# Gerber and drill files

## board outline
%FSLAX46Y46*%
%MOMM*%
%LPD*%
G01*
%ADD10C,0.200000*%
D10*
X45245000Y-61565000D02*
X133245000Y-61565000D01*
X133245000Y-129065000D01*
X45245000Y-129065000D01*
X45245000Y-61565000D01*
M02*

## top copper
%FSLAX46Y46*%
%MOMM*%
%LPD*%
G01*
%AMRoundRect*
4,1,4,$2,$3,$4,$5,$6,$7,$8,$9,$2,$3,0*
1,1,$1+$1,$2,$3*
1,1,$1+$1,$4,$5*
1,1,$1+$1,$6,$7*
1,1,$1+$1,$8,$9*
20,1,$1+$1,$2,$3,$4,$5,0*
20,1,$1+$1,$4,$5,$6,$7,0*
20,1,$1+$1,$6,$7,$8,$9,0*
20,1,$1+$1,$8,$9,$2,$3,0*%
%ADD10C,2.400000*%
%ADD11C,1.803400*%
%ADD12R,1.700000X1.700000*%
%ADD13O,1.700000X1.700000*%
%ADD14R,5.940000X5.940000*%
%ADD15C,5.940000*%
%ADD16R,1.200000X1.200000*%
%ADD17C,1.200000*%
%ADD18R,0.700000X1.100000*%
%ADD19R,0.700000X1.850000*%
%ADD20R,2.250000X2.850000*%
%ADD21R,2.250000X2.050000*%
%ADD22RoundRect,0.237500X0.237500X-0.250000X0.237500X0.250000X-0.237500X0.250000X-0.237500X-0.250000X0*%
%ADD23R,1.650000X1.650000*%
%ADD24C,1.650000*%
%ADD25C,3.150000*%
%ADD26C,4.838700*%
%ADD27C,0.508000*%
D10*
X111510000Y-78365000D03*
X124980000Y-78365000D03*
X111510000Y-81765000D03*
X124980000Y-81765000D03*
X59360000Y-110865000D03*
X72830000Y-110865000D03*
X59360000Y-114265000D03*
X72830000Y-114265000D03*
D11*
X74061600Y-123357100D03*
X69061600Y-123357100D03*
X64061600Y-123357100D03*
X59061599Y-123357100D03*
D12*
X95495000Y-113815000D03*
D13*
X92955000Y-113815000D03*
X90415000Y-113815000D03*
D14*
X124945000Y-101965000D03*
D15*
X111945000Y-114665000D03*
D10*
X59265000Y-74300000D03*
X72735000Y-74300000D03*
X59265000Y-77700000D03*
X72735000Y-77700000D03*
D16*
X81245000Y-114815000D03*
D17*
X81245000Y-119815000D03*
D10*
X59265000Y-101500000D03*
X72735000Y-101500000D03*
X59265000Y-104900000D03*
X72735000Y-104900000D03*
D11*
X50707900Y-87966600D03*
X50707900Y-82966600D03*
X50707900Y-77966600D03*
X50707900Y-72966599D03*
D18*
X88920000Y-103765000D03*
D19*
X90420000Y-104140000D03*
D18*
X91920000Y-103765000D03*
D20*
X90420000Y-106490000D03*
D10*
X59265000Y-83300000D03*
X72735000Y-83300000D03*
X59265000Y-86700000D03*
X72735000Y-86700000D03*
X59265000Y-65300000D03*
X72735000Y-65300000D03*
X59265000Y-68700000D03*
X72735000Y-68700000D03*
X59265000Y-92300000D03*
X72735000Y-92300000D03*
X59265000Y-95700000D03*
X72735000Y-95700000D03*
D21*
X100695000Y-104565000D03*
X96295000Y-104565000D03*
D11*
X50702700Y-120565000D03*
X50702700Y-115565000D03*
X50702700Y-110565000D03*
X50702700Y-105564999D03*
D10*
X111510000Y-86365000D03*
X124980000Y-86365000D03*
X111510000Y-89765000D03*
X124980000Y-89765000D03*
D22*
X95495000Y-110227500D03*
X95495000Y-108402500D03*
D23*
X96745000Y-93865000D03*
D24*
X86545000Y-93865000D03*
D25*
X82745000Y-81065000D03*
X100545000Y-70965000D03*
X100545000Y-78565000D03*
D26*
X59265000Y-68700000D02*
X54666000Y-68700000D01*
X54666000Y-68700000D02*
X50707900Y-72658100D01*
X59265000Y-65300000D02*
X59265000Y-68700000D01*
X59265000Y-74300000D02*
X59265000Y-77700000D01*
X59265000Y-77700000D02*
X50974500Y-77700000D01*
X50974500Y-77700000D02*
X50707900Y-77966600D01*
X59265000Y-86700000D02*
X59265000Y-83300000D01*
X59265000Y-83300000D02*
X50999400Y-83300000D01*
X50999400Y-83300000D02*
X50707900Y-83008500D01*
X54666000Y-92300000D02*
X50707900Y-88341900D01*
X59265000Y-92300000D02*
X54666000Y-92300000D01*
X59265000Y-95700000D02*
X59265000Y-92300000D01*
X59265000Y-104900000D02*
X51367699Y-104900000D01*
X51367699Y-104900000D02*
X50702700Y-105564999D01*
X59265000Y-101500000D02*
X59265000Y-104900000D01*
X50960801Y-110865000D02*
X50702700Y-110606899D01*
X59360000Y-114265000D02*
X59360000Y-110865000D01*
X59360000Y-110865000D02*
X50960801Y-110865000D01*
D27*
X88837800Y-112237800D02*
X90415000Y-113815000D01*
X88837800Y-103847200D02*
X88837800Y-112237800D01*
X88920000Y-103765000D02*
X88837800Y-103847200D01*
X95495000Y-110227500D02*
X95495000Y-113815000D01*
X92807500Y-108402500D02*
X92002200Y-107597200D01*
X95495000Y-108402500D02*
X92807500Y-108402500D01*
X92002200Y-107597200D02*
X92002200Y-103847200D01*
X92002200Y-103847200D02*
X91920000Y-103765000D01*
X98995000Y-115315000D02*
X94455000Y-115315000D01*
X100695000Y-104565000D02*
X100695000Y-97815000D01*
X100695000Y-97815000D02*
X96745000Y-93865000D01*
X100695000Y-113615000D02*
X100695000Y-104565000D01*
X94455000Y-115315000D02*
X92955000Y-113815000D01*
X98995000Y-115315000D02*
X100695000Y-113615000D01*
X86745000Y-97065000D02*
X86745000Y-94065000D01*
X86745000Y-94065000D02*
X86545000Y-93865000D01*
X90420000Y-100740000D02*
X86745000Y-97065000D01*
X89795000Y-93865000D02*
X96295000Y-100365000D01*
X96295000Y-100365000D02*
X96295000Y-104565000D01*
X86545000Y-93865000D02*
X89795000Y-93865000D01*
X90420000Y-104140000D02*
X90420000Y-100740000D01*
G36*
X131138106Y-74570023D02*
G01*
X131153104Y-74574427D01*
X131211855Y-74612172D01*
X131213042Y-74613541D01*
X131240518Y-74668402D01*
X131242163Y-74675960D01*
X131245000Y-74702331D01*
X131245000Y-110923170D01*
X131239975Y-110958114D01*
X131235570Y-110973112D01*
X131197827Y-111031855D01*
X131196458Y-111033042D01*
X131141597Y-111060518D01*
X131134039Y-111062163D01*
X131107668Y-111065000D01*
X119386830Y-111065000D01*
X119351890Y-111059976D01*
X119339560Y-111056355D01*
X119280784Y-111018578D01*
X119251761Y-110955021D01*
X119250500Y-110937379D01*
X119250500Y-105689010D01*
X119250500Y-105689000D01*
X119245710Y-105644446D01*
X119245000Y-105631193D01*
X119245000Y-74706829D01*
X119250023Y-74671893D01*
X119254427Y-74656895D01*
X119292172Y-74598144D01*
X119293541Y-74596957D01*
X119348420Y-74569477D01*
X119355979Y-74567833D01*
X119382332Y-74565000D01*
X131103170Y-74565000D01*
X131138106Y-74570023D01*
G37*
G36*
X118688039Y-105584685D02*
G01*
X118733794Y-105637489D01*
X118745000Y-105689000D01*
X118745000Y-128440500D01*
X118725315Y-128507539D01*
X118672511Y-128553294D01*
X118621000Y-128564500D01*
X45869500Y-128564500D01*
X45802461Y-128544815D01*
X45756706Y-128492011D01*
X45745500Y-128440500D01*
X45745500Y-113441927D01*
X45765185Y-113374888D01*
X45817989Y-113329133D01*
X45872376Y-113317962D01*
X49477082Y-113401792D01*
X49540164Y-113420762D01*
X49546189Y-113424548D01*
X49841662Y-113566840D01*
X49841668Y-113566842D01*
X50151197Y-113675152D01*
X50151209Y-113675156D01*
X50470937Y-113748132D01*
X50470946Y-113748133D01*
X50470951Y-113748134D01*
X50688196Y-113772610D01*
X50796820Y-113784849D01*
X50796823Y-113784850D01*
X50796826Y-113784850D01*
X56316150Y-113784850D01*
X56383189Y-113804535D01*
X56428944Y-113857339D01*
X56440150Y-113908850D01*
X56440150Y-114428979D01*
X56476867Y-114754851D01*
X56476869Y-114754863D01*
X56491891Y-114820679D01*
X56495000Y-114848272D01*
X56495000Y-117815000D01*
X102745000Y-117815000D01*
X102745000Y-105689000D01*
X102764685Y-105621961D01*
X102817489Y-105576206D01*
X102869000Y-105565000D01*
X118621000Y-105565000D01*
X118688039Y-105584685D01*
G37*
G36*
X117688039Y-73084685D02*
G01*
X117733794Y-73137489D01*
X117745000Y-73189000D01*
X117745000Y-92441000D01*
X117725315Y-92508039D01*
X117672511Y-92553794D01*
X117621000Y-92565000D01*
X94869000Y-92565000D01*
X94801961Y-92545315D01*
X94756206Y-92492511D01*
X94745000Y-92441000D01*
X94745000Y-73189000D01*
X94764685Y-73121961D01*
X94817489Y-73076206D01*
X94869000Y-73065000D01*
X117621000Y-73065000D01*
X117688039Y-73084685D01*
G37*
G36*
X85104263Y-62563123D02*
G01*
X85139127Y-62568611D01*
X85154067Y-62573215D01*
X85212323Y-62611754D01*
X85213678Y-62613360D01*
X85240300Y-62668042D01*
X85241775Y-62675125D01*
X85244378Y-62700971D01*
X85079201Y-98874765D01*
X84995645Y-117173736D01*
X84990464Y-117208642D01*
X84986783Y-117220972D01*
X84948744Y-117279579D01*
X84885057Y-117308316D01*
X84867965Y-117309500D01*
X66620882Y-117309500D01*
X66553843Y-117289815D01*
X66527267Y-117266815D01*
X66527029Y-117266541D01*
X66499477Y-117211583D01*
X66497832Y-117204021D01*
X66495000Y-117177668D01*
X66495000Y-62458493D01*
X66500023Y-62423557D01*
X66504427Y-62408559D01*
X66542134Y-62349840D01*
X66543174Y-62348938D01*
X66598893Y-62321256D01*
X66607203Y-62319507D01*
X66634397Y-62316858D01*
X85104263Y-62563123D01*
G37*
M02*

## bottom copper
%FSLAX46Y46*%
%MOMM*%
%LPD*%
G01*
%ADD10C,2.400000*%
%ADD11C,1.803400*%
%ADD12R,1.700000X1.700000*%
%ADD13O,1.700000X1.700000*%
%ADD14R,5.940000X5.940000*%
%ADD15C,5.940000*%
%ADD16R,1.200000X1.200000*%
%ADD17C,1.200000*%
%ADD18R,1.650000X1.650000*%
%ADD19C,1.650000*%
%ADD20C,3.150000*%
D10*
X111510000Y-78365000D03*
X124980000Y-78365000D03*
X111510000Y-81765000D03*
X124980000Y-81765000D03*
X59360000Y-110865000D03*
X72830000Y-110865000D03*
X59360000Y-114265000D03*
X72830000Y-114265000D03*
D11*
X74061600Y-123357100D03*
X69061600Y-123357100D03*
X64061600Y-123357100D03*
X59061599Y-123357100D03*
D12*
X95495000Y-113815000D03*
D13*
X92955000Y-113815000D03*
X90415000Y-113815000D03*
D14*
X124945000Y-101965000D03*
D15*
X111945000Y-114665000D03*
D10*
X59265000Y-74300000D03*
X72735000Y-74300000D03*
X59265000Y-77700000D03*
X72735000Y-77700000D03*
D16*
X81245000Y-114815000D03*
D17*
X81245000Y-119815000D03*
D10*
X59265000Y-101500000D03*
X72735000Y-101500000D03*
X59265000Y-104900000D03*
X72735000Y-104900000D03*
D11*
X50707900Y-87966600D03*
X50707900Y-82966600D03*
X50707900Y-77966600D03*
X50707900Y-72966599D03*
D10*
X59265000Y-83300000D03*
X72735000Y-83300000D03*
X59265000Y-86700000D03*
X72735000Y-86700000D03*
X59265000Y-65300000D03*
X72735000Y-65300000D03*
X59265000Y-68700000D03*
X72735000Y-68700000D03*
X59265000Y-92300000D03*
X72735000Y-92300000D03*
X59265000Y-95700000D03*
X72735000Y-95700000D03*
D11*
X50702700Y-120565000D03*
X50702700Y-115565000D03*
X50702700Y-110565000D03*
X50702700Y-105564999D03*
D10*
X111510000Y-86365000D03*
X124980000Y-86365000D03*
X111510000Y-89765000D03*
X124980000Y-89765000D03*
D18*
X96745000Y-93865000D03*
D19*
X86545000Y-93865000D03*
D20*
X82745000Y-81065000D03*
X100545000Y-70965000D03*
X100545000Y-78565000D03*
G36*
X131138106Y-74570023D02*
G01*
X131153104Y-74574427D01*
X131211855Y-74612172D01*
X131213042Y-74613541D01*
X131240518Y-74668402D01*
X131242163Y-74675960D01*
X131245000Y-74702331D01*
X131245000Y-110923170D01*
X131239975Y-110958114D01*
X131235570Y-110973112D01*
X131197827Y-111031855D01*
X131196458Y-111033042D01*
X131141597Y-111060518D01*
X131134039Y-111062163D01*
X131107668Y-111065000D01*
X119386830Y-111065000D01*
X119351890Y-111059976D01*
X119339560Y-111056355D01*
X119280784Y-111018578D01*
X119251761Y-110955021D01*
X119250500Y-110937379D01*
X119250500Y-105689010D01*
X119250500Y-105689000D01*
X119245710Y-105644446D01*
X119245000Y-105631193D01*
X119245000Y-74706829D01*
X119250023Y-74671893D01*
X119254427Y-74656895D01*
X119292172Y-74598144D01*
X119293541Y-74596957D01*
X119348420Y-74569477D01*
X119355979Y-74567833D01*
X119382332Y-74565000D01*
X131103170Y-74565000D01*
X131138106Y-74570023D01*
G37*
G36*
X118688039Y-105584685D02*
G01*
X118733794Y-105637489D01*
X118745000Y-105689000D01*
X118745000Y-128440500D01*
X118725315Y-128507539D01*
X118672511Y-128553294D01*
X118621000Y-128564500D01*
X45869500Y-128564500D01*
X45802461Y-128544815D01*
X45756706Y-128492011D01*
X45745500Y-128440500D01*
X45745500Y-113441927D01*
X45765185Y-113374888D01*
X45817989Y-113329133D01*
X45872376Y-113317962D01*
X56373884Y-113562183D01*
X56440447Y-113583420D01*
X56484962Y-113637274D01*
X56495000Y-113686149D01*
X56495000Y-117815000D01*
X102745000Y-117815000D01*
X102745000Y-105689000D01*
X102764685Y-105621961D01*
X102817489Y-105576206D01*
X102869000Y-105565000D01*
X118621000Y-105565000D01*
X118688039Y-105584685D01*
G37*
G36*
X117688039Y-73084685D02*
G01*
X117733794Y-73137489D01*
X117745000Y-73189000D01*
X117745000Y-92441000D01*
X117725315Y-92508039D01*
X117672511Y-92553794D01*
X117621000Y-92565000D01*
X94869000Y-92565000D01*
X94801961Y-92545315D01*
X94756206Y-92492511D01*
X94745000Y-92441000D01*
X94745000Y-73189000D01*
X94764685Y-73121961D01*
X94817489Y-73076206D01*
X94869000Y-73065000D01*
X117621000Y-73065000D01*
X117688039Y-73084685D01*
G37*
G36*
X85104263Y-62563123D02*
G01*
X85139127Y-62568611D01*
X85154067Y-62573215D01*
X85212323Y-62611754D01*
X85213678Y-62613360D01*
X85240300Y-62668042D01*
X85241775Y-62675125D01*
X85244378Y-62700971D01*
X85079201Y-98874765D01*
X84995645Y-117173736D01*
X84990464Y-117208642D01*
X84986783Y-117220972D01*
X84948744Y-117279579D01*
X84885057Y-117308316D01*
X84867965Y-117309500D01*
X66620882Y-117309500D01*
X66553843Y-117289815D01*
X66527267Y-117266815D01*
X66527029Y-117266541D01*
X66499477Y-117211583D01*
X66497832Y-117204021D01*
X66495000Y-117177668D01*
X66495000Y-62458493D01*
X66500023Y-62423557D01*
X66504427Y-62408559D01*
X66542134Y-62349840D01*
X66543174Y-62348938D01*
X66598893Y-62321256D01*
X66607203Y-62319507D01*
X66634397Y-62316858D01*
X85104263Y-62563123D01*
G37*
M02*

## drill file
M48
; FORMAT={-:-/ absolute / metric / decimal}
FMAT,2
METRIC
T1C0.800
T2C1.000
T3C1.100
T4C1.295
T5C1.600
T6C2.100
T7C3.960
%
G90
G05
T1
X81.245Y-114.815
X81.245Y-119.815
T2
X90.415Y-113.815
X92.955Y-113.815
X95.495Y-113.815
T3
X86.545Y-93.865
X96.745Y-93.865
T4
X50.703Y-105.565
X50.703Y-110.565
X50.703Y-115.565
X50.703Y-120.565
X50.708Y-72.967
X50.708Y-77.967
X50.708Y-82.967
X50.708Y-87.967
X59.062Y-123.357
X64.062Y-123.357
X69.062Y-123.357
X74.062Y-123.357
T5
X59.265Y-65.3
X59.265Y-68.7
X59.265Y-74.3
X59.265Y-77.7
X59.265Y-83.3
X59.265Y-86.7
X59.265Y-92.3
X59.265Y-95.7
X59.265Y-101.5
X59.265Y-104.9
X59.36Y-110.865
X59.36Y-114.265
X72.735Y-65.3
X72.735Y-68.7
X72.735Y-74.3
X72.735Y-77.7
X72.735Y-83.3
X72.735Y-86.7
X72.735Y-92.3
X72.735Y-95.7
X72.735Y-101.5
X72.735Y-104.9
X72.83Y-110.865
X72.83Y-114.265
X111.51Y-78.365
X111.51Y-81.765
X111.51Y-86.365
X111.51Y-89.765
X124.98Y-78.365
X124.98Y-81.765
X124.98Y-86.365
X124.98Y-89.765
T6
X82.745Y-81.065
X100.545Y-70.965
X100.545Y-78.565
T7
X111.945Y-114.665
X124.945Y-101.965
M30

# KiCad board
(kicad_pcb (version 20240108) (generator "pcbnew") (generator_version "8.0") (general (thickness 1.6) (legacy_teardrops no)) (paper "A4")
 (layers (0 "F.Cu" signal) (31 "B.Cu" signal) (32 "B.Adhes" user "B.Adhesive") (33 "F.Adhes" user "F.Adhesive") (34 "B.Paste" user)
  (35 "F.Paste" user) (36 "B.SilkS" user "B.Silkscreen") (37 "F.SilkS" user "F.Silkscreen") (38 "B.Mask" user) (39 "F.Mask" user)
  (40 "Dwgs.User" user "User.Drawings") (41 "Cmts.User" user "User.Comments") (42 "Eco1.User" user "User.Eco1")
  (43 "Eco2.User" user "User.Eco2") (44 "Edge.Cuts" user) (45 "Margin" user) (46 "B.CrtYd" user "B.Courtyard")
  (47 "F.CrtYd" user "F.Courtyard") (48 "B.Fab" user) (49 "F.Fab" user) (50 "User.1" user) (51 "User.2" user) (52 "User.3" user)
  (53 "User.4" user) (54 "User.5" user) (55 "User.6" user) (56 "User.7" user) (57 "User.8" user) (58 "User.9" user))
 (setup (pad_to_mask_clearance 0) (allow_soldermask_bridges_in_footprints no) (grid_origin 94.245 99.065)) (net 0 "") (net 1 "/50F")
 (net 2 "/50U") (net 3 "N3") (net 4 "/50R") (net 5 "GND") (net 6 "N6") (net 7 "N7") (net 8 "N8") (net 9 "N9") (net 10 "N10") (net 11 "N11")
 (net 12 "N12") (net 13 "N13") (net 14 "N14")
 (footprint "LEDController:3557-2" (layer "F.Cu") (at 118.245 80.065)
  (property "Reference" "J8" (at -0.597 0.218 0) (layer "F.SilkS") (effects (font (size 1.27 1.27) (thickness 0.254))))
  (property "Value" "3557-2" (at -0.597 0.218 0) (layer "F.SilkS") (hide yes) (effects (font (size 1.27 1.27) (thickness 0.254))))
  (pad "1" thru_hole circle (at -6.735 -1.7) (size 2.4 2.4) (drill 1.6) (layers "*.Cu" "*.Mask") (remove_unused_layers no) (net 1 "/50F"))
  (pad "2" thru_hole circle (at 6.735 -1.7) (size 2.4 2.4) (drill 1.6) (layers "*.Cu" "*.Mask") (remove_unused_layers no) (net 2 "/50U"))
  (pad "3" thru_hole circle (at -6.735 1.7) (size 2.4 2.4) (drill 1.6) (layers "*.Cu" "*.Mask") (remove_unused_layers no) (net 1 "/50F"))
  (pad "4" thru_hole circle (at 6.735 1.7) (size 2.4 2.4) (drill 1.6) (layers "*.Cu" "*.Mask") (remove_unused_layers no) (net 2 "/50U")))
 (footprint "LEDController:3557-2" (layer "F.Cu") (at 66.095 112.565)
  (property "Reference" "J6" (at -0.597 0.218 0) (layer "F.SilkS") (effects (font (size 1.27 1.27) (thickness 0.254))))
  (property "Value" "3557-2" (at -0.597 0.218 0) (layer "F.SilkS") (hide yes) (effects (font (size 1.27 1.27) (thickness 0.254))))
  (pad "1" thru_hole circle (at -6.735 -1.7) (size 2.4 2.4) (drill 1.6) (layers "*.Cu" "*.Mask") (remove_unused_layers no) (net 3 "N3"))
  (pad "2" thru_hole circle (at 6.735 -1.7) (size 2.4 2.4) (drill 1.6) (layers "*.Cu" "*.Mask") (remove_unused_layers no) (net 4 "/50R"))
  (pad "3" thru_hole circle (at -6.735 1.7) (size 2.4 2.4) (drill 1.6) (layers "*.Cu" "*.Mask") (remove_unused_layers no) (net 3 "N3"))
  (pad "4" thru_hole circle (at 6.735 1.7) (size 2.4 2.4) (drill 1.6) (layers "*.Cu" "*.Mask") (remove_unused_layers no) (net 4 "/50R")))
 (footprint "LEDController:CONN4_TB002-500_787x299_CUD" (layer "F.Cu") (at 74.0616 123.3571)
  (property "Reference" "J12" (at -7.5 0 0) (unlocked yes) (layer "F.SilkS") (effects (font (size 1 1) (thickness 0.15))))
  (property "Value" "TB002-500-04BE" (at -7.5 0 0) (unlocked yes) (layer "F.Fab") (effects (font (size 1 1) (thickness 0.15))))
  (pad "1" thru_hole circle (at 0 0) (size 1.8034 1.8034) (drill 1.2954) (layers "*.Cu" "*.Mask") (remove_unused_layers no) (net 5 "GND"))
  (pad "2" thru_hole circle (at -5 0) (size 1.8034 1.8034) (drill 1.2954) (layers "*.Cu" "*.Mask") (remove_unused_layers no) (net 5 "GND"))
  (pad "3" thru_hole circle (at -10 0) (size 1.8034 1.8034) (drill 1.2954) (layers "*.Cu" "*.Mask") (remove_unused_layers no) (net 5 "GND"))
  (pad "4" thru_hole circle (at -15.000001 0) (size 1.8034 1.8034) (drill 1.2954) (layers "*.Cu" "*.Mask") (remove_unused_layers no)
   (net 5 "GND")))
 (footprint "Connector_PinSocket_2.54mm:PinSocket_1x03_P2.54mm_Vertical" (layer "F.Cu") (at 95.495 113.815 -90)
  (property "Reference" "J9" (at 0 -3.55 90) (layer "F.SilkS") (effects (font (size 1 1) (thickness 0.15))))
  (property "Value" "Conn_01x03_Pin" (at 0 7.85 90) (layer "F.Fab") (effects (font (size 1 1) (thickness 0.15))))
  (pad "1" thru_hole rect (at 0 0 270) (size 1.7 1.7) (drill 1) (layers "*.Cu" "*.Mask") (remove_unused_layers no) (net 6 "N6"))
  (pad "2" thru_hole oval (at 0 2.54 270) (size 1.7 1.7) (drill 1) (layers "*.Cu" "*.Mask") (remove_unused_layers no) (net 1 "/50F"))
  (pad "3" thru_hole oval (at 0 5.08 270) (size 1.7 1.7) (drill 1) (layers "*.Cu" "*.Mask") (remove_unused_layers no) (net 5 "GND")))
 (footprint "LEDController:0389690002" (layer "F.Cu") (at 124.945 101.965 -90)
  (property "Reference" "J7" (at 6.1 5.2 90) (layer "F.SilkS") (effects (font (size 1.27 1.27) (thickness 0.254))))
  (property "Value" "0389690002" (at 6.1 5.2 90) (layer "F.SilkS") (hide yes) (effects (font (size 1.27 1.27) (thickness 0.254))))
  (pad "1" thru_hole rect (at 0 0 270) (size 5.94 5.94) (drill 3.96) (layers "*.Cu" "*.Mask") (remove_unused_layers no) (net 2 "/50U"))
  (pad "2" thru_hole circle (at 12.7 13 270) (size 5.94 5.94) (drill 3.96) (layers "*.Cu" "*.Mask") (remove_unused_layers no) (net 5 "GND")))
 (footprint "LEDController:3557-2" (layer "F.Cu") (at 66 76)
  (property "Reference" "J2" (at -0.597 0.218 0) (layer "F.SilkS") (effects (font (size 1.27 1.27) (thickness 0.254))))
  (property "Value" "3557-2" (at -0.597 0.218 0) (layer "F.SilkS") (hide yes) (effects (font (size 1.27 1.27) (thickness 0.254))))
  (pad "1" thru_hole circle (at -6.735 -1.7) (size 2.4 2.4) (drill 1.6) (layers "*.Cu" "*.Mask") (remove_unused_layers no) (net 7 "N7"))
  (pad "2" thru_hole circle (at 6.735 -1.7) (size 2.4 2.4) (drill 1.6) (layers "*.Cu" "*.Mask") (remove_unused_layers no) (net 4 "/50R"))
  (pad "3" thru_hole circle (at -6.735 1.7) (size 2.4 2.4) (drill 1.6) (layers "*.Cu" "*.Mask") (remove_unused_layers no) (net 7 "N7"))
  (pad "4" thru_hole circle (at 6.735 1.7) (size 2.4 2.4) (drill 1.6) (layers "*.Cu" "*.Mask") (remove_unused_layers no) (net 4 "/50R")))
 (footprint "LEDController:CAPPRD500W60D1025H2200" (layer "F.Cu") (at 81.245 114.815 -90)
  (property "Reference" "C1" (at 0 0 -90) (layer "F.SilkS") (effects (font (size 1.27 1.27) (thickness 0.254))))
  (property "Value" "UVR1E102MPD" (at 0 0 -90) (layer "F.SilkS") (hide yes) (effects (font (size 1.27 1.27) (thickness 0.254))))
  (pad "1" thru_hole rect (at 0 0 270) (size 1.2 1.2) (drill 0.8) (layers "*.Cu" "*.Mask") (remove_unused_layers no) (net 4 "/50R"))
  (pad "2" thru_hole circle (at 5 0 270) (size 1.2 1.2) (drill 0.8) (layers "*.Cu" "*.Mask") (remove_unused_layers no) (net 5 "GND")))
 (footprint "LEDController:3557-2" (layer "F.Cu") (at 66 103.2)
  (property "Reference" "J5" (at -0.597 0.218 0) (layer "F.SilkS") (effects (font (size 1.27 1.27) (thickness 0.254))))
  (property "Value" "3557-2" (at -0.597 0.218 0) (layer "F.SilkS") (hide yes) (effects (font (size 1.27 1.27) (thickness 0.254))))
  (pad "1" thru_hole circle (at -6.735 -1.7) (size 2.4 2.4) (drill 1.6) (layers "*.Cu" "*.Mask") (remove_unused_layers no) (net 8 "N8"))
  (pad "2" thru_hole circle (at 6.735 -1.7) (size 2.4 2.4) (drill 1.6) (layers "*.Cu" "*.Mask") (remove_unused_layers no) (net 4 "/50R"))
  (pad "3" thru_hole circle (at -6.735 1.7) (size 2.4 2.4) (drill 1.6) (layers "*.Cu" "*.Mask") (remove_unused_layers no) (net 8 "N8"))
  (pad "4" thru_hole circle (at 6.735 1.7) (size 2.4 2.4) (drill 1.6) (layers "*.Cu" "*.Mask") (remove_unused_layers no) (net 4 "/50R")))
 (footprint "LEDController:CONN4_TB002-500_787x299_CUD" (layer "F.Cu") (at 50.7079 87.9666 -90)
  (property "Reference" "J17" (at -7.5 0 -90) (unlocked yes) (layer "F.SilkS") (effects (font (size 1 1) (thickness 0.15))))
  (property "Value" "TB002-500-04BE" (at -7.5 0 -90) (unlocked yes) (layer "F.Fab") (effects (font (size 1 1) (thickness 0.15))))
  (pad "1" thru_hole circle (at 0 0 270) (size 1.8034 1.8034) (drill 1.2954) (layers "*.Cu" "*.Mask") (remove_unused_layers no) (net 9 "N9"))
  (pad "2" thru_hole circle (at -5 0 270) (size 1.8034 1.8034) (drill 1.2954) (layers "*.Cu" "*.Mask") (remove_unused_layers no)
   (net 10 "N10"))
  (pad "3" thru_hole circle (at -10 0 270) (size 1.8034 1.8034) (drill 1.2954) (layers "*.Cu" "*.Mask") (remove_unused_layers no)
   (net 7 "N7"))
  (pad "4" thru_hole circle (at -15.000001 0 270) (size 1.8034 1.8034) (drill 1.2954) (layers "*.Cu" "*.Mask") (remove_unused_layers no)
   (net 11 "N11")))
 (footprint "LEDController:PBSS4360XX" (layer "F.Cu") (at 90.42 105.565 180)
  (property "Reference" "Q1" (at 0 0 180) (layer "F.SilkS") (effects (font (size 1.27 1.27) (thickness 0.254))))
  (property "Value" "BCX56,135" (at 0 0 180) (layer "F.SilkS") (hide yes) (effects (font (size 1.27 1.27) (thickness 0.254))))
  (pad "1" smd rect (at 1.5 1.8 180) (size 0.7 1.1) (layers "F.Cu" "F.Paste" "F.Mask") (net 5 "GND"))
  (pad "2" smd rect (at 0 1.425 180) (size 0.7 1.85) (layers "F.Cu" "F.Paste" "F.Mask") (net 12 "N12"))
  (pad "3" smd rect (at -1.5 1.8 180) (size 0.7 1.1) (layers "F.Cu" "F.Paste" "F.Mask") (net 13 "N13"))
  (pad "4" smd rect (at 0 -0.925 180) (size 2.25 2.85) (layers "F.Cu" "F.Paste" "F.Mask") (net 12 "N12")))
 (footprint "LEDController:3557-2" (layer "F.Cu") (at 66 85)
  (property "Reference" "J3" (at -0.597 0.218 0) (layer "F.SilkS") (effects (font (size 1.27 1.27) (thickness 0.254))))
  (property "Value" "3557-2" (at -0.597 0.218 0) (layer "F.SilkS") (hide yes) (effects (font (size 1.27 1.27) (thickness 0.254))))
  (pad "1" thru_hole circle (at -6.735 -1.7) (size 2.4 2.4) (drill 1.6) (layers "*.Cu" "*.Mask") (remove_unused_layers no) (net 10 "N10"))
  (pad "2" thru_hole circle (at 6.735 -1.7) (size 2.4 2.4) (drill 1.6) (layers "*.Cu" "*.Mask") (remove_unused_layers no) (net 4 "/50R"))
  (pad "3" thru_hole circle (at -6.735 1.7) (size 2.4 2.4) (drill 1.6) (layers "*.Cu" "*.Mask") (remove_unused_layers no) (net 10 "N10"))
  (pad "4" thru_hole circle (at 6.735 1.7) (size 2.4 2.4) (drill 1.6) (layers "*.Cu" "*.Mask") (remove_unused_layers no) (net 4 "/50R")))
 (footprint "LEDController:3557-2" (layer "F.Cu") (at 66 67)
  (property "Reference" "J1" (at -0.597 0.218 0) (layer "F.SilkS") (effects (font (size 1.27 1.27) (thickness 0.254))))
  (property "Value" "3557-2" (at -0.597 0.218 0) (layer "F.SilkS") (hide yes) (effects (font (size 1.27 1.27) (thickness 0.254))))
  (pad "1" thru_hole circle (at -6.735 -1.7) (size 2.4 2.4) (drill 1.6) (layers "*.Cu" "*.Mask") (remove_unused_layers no) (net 11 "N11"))
  (pad "2" thru_hole circle (at 6.735 -1.7) (size 2.4 2.4) (drill 1.6) (layers "*.Cu" "*.Mask") (remove_unused_layers no) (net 4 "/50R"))
  (pad "3" thru_hole circle (at -6.735 1.7) (size 2.4 2.4) (drill 1.6) (layers "*.Cu" "*.Mask") (remove_unused_layers no) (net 11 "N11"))
  (pad "4" thru_hole circle (at 6.735 1.7) (size 2.4 2.4) (drill 1.6) (layers "*.Cu" "*.Mask") (remove_unused_layers no) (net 4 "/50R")))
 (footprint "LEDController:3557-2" (layer "F.Cu") (at 66 94)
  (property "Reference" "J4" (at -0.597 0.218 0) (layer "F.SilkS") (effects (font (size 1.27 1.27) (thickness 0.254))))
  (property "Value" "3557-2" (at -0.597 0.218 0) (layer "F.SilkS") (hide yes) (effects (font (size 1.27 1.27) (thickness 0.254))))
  (pad "1" thru_hole circle (at -6.735 -1.7) (size 2.4 2.4) (drill 1.6) (layers "*.Cu" "*.Mask") (remove_unused_layers no) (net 9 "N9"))
  (pad "2" thru_hole circle (at 6.735 -1.7) (size 2.4 2.4) (drill 1.6) (layers "*.Cu" "*.Mask") (remove_unused_layers no) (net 4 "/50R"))
  (pad "3" thru_hole circle (at -6.735 1.7) (size 2.4 2.4) (drill 1.6) (layers "*.Cu" "*.Mask") (remove_unused_layers no) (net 9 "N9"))
  (pad "4" thru_hole circle (at 6.735 1.7) (size 2.4 2.4) (drill 1.6) (layers "*.Cu" "*.Mask") (remove_unused_layers no) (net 4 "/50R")))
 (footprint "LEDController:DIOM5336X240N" (layer "F.Cu") (at 98.495 104.565 180)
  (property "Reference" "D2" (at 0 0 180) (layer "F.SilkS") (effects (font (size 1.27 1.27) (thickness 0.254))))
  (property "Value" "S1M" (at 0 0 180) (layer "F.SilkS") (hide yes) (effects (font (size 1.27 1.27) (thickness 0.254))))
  (pad "1" smd rect (at -2.2 0 270) (size 2.05 2.25) (layers "F.Cu" "F.Paste" "F.Mask") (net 1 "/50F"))
  (pad "2" smd rect (at 2.2 0 270) (size 2.05 2.25) (layers "F.Cu" "F.Paste" "F.Mask") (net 12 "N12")))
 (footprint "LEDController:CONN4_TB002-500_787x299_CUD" (layer "F.Cu") (at 50.7027 120.565 -90)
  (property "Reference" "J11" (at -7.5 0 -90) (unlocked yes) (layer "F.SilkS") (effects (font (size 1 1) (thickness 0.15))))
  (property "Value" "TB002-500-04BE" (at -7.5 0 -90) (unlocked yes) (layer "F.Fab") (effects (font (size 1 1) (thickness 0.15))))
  (pad "1" thru_hole circle (at 0 0 270) (size 1.8034 1.8034) (drill 1.2954) (layers "*.Cu" "*.Mask") (remove_unused_layers no)
   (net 5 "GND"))
  (pad "2" thru_hole circle (at -5 0 270) (size 1.8034 1.8034) (drill 1.2954) (layers "*.Cu" "*.Mask") (remove_unused_layers no)
   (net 5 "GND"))
  (pad "3" thru_hole circle (at -10 0 270) (size 1.8034 1.8034) (drill 1.2954) (layers "*.Cu" "*.Mask") (remove_unused_layers no)
   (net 3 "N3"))
  (pad "4" thru_hole circle (at -15.000001 0 270) (size 1.8034 1.8034) (drill 1.2954) (layers "*.Cu" "*.Mask") (remove_unused_layers no)
   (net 8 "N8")))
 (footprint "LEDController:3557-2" (layer "F.Cu") (at 118.245 88.065)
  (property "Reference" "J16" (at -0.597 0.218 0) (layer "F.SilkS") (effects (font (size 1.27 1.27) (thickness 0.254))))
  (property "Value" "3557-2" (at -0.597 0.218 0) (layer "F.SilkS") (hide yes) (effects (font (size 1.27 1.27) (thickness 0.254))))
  (pad "1" thru_hole circle (at -6.735 -1.7) (size 2.4 2.4) (drill 1.6) (layers "*.Cu" "*.Mask") (remove_unused_layers no) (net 1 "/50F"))
  (pad "2" thru_hole circle (at 6.735 -1.7) (size 2.4 2.4) (drill 1.6) (layers "*.Cu" "*.Mask") (remove_unused_layers no) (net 2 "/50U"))
  (pad "3" thru_hole circle (at -6.735 1.7) (size 2.4 2.4) (drill 1.6) (layers "*.Cu" "*.Mask") (remove_unused_layers no) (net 1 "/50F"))
  (pad "4" thru_hole circle (at 6.735 1.7) (size 2.4 2.4) (drill 1.6) (layers "*.Cu" "*.Mask") (remove_unused_layers no) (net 2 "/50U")))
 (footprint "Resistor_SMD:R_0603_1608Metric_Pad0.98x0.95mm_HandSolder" (layer "F.Cu") (at 95.495 109.315 90)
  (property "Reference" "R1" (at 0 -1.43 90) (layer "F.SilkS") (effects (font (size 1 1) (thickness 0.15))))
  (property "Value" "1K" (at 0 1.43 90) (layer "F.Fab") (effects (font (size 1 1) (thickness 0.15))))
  (pad "1" smd roundrect (at -0.9125 0 90) (size 0.975 0.95) (layers "F.Cu" "F.Paste" "F.Mask") (roundrect_rratio 0.25) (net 6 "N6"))
  (pad "2" smd roundrect (at 0.9125 0 90) (size 0.975 0.95) (layers "F.Cu" "F.Paste" "F.Mask") (roundrect_rratio 0.25) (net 13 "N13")))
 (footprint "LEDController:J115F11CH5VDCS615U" (layer "F.Cu") (at 96.745 93.865)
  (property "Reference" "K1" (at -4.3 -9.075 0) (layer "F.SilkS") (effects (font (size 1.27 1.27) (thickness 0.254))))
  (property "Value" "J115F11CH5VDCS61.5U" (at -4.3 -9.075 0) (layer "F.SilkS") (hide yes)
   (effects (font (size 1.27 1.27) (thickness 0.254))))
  (pad "1" thru_hole rect (at 0 0) (size 1.65 1.65) (drill 1.1) (layers "*.Cu" "*.Mask") (remove_unused_layers no) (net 1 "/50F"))
  (pad "2" thru_hole circle (at -10.2 0) (size 1.65 1.65) (drill 1.1) (layers "*.Cu" "*.Mask") (remove_unused_layers no) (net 12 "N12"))
  (pad "3" thru_hole circle (at -14 -12.8) (size 3.15 3.15) (drill 2.1) (layers "*.Cu" "*.Mask") (remove_unused_layers no) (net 4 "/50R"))
  (pad "4" thru_hole circle (at 3.8 -22.9) (size 3.15 3.15) (drill 2.1) (layers "*.Cu" "*.Mask") (remove_unused_layers no) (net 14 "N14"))
  (pad "5" thru_hole circle (at 3.8 -15.3) (size 3.15 3.15) (drill 2.1) (layers "*.Cu" "*.Mask") (remove_unused_layers no) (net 1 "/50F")))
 (gr_rect (start 45.245 61.565) (end 133.245 129.065) (stroke (width 0.2) (type default)) (fill none) (layer "Edge.Cuts"))
 (segment (start 59.265 68.7) (end 54.666 68.7) (width 4.8387) (layer "F.Cu") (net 11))
 (segment (start 54.666 68.7) (end 50.7079 72.6581) (width 4.8387) (layer "F.Cu") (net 11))
 (segment (start 59.265 65.3) (end 59.265 68.7) (width 4.8387) (layer "F.Cu") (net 11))
 (segment (start 59.265 74.3) (end 59.265 77.7) (width 4.8387) (layer "F.Cu") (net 7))
 (segment (start 59.265 77.7) (end 50.9745 77.7) (width 4.8387) (layer "F.Cu") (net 7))
 (segment (start 50.9745 77.7) (end 50.7079 77.9666) (width 4.8387) (layer "F.Cu") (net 7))
 (segment (start 59.265 86.7) (end 59.265 83.3) (width 4.8387) (layer "F.Cu") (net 10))
 (segment (start 59.265 83.3) (end 50.9994 83.3) (width 4.8387) (layer "F.Cu") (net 10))
 (segment (start 50.9994 83.3) (end 50.7079 83.0085) (width 4.8387) (layer "F.Cu") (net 10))
 (segment (start 54.666 92.3) (end 50.7079 88.3419) (width 4.8387) (layer "F.Cu") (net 9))
 (segment (start 59.265 92.3) (end 54.666 92.3) (width 4.8387) (layer "F.Cu") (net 9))
 (segment (start 59.265 95.7) (end 59.265 92.3) (width 4.8387) (layer "F.Cu") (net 9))
 (segment (start 59.265 104.9) (end 51.367699 104.9) (width 4.8387) (layer "F.Cu") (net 8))
 (segment (start 51.367699 104.9) (end 50.7027 105.564999) (width 4.8387) (layer "F.Cu") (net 8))
 (segment (start 59.265 101.5) (end 59.265 104.9) (width 4.8387) (layer "F.Cu") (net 8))
 (segment (start 50.960801 110.865) (end 50.7027 110.606899) (width 4.8387) (layer "F.Cu") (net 3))
 (segment (start 59.36 114.265) (end 59.36 110.865) (width 4.8387) (layer "F.Cu") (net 3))
 (segment (start 59.36 110.865) (end 50.960801 110.865) (width 4.8387) (layer "F.Cu") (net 3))
 (segment (start 88.8378 112.2378) (end 90.415 113.815) (width 0.508) (layer "F.Cu") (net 5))
 (segment (start 88.8378 103.8472) (end 88.8378 112.2378) (width 0.508) (layer "F.Cu") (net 5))
 (segment (start 88.92 103.765) (end 88.8378 103.8472) (width 0.508) (layer "F.Cu") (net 5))
 (segment (start 95.495 110.2275) (end 95.495 113.815) (width 0.508) (layer "F.Cu") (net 6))
 (segment (start 92.8075 108.4025) (end 92.0022 107.5972) (width 0.508) (layer "F.Cu") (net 13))
 (segment (start 95.495 108.4025) (end 92.8075 108.4025) (width 0.508) (layer "F.Cu") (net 13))
 (segment (start 92.0022 107.5972) (end 92.0022 103.8472) (width 0.508) (layer "F.Cu") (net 13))
 (segment (start 92.0022 103.8472) (end 91.92 103.765) (width 0.508) (layer "F.Cu") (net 13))
 (segment (start 98.995 115.315) (end 94.455 115.315) (width 0.508) (layer "F.Cu") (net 1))
 (segment (start 100.695 104.565) (end 100.695 97.815) (width 0.508) (layer "F.Cu") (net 1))
 (segment (start 100.695 97.815) (end 96.745 93.865) (width 0.508) (layer "F.Cu") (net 1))
 (segment (start 100.695 113.615) (end 100.695 104.565) (width 0.508) (layer "F.Cu") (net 1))
 (segment (start 94.455 115.315) (end 92.955 113.815) (width 0.508) (layer "F.Cu") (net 1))
 (segment (start 98.995 115.315) (end 100.695 113.615) (width 0.508) (layer "F.Cu") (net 1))
 (segment (start 86.745 97.065) (end 86.745 94.065) (width 0.508) (layer "F.Cu") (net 12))
 (segment (start 86.745 94.065) (end 86.545 93.865) (width 0.508) (layer "F.Cu") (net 12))
 (segment (start 90.42 100.74) (end 86.745 97.065) (width 0.508) (layer "F.Cu") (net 12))
 (segment (start 89.795 93.865) (end 96.295 100.365) (width 0.508) (layer "F.Cu") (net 12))
 (segment (start 96.295 100.365) (end 96.295 104.565) (width 0.508) (layer "F.Cu") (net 12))
 (segment (start 86.545 93.865) (end 89.795 93.865) (width 0.508) (layer "F.Cu") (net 12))
 (segment (start 90.42 104.14) (end 90.42 100.74) (width 0.508) (layer "F.Cu") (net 12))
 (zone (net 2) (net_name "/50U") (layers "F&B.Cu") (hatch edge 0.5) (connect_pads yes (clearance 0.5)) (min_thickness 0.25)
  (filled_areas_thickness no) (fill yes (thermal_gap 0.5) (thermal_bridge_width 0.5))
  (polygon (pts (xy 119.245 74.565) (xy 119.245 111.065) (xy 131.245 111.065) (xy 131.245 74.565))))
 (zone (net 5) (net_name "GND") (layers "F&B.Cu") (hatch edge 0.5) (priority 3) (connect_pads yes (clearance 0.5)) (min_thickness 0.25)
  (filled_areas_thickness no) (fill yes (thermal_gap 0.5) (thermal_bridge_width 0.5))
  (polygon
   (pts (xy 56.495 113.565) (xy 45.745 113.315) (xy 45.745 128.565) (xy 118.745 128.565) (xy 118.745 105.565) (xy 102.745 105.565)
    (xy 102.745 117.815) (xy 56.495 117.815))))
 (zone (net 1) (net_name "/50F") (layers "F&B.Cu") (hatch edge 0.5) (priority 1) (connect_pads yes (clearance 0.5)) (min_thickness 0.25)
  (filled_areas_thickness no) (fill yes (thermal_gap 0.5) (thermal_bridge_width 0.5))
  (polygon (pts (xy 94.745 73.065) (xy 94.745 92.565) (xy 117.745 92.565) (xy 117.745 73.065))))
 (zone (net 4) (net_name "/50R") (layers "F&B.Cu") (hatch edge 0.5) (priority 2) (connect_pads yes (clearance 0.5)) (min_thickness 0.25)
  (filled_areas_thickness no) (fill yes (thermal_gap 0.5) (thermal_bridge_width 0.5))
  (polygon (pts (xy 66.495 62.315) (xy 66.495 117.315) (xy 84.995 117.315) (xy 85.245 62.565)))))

